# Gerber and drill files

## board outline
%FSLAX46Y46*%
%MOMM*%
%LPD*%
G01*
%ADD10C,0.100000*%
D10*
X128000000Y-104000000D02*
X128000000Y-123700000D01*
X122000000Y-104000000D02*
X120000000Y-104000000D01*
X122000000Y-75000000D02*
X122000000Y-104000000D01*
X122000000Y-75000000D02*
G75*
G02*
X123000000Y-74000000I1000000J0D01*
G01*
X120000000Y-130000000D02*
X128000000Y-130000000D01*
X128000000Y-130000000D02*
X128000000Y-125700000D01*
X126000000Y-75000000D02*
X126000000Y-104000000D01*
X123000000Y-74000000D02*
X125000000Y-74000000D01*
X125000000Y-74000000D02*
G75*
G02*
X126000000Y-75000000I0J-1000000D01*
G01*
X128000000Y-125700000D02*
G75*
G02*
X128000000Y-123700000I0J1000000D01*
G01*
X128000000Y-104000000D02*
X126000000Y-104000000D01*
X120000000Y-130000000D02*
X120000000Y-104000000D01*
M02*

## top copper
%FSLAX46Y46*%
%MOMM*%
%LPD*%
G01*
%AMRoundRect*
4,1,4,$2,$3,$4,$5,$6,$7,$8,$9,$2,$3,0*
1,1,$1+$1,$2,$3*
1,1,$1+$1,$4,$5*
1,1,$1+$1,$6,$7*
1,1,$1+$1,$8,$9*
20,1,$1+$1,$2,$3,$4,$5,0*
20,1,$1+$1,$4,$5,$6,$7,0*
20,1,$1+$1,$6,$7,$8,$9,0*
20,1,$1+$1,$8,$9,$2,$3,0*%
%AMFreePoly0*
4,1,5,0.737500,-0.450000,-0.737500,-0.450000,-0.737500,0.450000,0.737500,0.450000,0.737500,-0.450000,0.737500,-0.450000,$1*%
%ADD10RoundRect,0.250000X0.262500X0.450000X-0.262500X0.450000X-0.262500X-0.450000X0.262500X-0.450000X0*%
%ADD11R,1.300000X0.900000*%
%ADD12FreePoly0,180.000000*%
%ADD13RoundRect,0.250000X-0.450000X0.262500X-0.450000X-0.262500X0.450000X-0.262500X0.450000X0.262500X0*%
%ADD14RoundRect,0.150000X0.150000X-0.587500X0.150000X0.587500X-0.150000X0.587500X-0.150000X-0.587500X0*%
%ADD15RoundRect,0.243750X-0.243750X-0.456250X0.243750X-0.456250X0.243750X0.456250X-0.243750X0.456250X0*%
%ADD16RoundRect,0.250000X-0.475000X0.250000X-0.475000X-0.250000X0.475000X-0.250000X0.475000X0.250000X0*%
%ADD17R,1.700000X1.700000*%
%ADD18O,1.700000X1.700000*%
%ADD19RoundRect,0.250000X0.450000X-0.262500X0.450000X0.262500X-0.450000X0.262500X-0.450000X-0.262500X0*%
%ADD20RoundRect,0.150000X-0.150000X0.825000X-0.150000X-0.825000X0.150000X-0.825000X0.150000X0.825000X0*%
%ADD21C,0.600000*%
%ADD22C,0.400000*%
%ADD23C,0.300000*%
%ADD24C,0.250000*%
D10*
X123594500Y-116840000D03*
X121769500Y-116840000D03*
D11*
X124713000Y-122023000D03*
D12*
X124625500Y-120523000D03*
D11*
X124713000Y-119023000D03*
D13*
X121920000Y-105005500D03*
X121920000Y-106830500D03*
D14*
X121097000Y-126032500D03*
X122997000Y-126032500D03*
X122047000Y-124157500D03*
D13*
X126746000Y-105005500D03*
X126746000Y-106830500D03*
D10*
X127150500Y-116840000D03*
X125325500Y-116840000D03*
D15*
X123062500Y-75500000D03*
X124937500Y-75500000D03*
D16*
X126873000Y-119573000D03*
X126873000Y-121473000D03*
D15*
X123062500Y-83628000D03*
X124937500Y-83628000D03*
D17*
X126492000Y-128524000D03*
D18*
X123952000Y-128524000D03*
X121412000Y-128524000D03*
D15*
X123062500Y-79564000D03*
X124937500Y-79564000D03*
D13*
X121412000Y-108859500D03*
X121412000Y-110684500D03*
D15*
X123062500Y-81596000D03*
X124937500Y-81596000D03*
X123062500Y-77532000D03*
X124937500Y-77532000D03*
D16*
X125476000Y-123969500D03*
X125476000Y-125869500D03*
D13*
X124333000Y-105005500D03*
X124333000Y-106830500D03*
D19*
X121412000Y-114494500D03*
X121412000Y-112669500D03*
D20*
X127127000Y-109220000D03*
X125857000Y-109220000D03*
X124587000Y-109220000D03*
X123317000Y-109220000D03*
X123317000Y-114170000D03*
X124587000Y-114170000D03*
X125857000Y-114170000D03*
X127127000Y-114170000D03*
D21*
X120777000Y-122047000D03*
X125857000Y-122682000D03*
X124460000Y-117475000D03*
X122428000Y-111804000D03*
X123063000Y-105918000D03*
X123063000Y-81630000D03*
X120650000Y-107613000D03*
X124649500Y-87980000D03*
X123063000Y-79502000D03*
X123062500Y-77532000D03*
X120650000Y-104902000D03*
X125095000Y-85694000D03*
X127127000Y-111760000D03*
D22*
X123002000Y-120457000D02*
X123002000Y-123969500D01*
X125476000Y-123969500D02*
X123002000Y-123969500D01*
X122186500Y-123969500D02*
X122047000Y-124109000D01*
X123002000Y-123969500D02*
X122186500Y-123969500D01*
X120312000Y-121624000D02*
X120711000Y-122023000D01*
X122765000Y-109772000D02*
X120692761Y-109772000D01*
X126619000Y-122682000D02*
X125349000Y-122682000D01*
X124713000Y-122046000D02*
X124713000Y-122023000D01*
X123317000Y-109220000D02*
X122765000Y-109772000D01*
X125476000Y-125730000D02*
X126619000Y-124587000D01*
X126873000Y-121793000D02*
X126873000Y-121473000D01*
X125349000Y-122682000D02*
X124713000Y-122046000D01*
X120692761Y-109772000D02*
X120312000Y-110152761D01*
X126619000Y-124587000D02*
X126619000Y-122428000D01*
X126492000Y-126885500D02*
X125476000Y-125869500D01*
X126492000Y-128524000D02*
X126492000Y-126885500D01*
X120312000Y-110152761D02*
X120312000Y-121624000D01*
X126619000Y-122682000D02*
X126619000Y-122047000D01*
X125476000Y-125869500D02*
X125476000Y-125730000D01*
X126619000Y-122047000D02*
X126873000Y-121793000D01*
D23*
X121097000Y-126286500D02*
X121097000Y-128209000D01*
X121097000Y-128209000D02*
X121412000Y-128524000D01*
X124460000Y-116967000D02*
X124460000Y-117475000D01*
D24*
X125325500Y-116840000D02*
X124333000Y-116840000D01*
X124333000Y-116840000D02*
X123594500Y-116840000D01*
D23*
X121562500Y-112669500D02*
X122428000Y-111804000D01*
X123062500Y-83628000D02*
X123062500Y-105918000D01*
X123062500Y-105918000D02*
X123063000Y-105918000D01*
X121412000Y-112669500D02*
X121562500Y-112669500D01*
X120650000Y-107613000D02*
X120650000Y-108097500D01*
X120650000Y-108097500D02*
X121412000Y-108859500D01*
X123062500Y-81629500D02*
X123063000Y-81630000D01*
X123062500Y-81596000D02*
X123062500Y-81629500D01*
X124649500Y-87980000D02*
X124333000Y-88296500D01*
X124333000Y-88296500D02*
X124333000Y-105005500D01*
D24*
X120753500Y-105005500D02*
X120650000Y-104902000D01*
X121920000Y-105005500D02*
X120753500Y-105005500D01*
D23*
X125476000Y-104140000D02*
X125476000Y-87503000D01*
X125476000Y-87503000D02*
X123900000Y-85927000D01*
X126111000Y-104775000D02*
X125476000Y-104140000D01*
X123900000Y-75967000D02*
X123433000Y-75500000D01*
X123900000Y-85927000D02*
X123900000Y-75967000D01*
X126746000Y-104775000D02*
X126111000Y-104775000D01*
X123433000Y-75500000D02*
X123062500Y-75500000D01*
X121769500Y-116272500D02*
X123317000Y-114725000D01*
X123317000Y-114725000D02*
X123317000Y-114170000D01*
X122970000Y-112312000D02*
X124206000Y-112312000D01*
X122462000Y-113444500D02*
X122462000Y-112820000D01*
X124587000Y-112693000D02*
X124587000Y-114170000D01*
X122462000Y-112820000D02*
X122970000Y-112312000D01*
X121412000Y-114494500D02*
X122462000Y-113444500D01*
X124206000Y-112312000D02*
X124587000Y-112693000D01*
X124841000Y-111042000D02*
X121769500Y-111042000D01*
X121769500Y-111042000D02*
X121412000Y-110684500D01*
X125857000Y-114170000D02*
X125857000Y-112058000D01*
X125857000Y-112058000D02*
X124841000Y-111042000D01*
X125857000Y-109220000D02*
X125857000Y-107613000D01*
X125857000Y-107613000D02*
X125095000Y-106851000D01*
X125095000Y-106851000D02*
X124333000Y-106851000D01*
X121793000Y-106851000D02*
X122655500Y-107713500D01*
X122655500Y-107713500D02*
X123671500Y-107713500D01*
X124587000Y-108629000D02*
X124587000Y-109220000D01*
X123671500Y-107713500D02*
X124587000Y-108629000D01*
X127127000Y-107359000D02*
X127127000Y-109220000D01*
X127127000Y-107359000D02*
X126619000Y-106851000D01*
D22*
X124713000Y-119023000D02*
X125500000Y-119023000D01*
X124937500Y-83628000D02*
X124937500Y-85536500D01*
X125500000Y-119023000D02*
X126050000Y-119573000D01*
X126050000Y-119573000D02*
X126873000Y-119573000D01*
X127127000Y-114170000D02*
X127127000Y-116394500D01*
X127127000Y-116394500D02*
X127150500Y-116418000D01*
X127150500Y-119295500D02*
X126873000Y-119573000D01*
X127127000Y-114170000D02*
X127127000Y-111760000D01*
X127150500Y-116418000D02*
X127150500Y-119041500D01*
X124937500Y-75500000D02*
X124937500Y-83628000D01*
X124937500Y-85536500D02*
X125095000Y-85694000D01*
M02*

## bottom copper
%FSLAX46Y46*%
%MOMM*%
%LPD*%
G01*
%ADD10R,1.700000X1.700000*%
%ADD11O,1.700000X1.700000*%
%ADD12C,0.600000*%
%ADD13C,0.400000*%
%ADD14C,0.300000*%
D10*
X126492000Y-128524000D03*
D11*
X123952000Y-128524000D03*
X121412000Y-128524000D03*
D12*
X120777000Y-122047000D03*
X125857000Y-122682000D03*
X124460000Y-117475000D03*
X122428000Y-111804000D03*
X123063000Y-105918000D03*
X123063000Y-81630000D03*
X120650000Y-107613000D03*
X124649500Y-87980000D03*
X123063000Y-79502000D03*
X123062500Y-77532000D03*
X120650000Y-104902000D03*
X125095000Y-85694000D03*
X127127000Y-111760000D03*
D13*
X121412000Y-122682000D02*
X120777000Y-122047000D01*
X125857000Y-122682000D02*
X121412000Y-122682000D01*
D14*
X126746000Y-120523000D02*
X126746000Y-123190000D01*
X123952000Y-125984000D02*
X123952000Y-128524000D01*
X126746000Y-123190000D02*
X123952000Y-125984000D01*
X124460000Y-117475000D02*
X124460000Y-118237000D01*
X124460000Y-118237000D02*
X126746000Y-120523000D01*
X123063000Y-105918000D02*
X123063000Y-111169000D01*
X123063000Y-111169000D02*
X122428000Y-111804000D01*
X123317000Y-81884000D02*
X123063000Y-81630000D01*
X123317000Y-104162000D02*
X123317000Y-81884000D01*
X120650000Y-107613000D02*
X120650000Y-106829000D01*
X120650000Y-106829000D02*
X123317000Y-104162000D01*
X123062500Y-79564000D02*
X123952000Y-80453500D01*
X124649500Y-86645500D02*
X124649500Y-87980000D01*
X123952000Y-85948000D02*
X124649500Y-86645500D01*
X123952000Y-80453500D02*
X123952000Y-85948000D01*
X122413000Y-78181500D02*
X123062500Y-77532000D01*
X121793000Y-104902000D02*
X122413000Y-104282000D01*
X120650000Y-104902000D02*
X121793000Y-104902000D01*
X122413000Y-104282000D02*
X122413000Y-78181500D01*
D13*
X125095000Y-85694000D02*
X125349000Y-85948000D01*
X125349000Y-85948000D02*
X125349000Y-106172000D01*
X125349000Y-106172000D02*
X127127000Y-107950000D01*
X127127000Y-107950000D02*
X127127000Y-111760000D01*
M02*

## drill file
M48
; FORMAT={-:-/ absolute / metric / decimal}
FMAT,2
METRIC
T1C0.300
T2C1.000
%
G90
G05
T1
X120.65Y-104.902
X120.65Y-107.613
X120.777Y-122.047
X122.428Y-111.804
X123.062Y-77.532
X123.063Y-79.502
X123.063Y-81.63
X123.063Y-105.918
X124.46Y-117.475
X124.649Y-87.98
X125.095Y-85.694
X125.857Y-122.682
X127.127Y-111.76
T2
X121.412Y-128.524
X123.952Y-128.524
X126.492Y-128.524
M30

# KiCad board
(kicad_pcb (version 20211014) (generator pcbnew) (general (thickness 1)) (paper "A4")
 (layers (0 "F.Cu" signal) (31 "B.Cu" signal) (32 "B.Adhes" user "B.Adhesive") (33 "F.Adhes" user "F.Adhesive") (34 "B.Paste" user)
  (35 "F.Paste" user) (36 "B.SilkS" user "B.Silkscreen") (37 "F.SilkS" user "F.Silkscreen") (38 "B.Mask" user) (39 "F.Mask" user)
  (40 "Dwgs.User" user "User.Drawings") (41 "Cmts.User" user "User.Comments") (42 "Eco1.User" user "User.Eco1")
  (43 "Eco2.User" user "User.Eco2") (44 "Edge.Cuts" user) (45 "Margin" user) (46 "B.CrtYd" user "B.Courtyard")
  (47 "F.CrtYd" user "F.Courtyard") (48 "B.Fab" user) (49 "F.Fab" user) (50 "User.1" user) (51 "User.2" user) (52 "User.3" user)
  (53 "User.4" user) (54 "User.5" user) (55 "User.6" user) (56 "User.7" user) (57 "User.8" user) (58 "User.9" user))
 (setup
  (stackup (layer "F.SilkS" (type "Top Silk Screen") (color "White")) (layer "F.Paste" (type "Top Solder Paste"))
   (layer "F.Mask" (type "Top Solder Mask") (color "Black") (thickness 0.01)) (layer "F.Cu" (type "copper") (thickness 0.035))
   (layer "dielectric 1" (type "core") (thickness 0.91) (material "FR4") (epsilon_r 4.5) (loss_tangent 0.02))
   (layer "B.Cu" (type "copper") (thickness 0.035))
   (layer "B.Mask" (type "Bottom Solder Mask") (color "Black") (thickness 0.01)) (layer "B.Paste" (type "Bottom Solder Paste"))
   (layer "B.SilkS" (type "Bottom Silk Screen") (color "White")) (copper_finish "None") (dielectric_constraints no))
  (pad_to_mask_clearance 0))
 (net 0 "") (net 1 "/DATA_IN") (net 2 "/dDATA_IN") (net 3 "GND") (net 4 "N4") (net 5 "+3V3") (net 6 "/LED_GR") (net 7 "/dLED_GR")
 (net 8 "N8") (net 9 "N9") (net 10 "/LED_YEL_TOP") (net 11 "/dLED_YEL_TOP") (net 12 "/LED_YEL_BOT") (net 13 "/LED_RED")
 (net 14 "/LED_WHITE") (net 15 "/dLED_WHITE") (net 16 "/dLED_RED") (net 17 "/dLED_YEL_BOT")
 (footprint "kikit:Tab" (layer "F.Cu") (at 126.238 84.455 180)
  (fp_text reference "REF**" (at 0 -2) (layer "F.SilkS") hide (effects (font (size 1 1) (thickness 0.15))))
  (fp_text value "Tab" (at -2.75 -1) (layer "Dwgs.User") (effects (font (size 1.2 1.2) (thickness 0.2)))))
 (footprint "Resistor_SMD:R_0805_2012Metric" (layer "F.Cu") (at 122.682 116.84 180)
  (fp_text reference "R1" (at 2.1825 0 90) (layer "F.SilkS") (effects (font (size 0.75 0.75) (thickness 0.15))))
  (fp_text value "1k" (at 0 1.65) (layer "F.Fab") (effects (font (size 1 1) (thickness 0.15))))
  (pad "1" smd roundrect (at -0.9125 0 180) (size 1.025 1.4) (layers "F.Cu" "F.Paste" "F.Mask") (roundrect_rratio 0.243902)
   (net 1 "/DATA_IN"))
  (pad "2" smd roundrect (at 0.9125 0 180) (size 1.025 1.4) (layers "F.Cu" "F.Paste" "F.Mask") (roundrect_rratio 0.243902)
   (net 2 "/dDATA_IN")))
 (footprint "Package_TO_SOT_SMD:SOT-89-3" (layer "F.Cu") (at 123.063 120.523 180)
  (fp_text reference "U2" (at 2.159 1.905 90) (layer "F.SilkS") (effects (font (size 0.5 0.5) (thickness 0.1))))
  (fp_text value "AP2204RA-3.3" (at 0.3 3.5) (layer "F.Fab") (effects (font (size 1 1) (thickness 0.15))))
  (pad "1" smd rect (at -1.65 -1.5 180) (size 1.3 0.9) (layers "F.Cu" "F.Paste" "F.Mask") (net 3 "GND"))
  (pad "2" smd custom (at -1.5625 0 180) (size 1.475 0.9) (layers "F.Cu" "F.Paste" "F.Mask") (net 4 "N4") (zone_connect 2)
   (options (clearance outline) (anchor rect)) (primitives))
  (pad "3" smd rect (at -1.65 1.5 180) (size 1.3 0.9) (layers "F.Cu" "F.Paste" "F.Mask") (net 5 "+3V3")))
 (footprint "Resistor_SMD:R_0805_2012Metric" (layer "F.Cu") (at 121.92 105.918 -90)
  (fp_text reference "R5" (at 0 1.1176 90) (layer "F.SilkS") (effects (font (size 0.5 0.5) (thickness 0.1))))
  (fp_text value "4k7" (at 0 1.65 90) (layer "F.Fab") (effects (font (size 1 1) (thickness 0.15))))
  (pad "1" smd roundrect (at -0.9125 0 270) (size 1.025 1.4) (layers "F.Cu" "F.Paste" "F.Mask") (roundrect_rratio 0.243902)
   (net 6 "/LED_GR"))
  (pad "2" smd roundrect (at 0.9125 0 270) (size 1.025 1.4) (layers "F.Cu" "F.Paste" "F.Mask") (roundrect_rratio 0.243902)
   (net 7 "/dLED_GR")))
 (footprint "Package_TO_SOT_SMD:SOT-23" (layer "F.Cu") (at 122.047 125.095 90)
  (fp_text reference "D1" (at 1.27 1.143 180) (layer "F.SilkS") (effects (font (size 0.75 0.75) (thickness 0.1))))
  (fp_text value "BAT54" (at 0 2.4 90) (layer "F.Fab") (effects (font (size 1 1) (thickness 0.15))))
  (pad "1" smd roundrect (at -0.9375 -0.95 90) (size 1.475 0.6) (layers "F.Cu" "F.Paste" "F.Mask") (roundrect_rratio 0.25) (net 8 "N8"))
  (pad "2" smd roundrect (at -0.9375 0.95 90) (size 1.475 0.6) (layers "F.Cu" "F.Paste" "F.Mask") (roundrect_rratio 0.25) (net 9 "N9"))
  (pad "3" smd roundrect (at 0.9375 0 90) (size 1.475 0.6) (layers "F.Cu" "F.Paste" "F.Mask") (roundrect_rratio 0.25) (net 4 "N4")))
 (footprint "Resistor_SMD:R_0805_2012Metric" (layer "F.Cu") (at 126.746 105.918 -90)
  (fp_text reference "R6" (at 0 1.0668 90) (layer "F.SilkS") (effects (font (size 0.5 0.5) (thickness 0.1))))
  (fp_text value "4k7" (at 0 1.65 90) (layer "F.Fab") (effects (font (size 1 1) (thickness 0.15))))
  (pad "1" smd roundrect (at -0.9125 0 270) (size 1.025 1.4) (layers "F.Cu" "F.Paste" "F.Mask") (roundrect_rratio 0.243902)
   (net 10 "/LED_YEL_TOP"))
  (pad "2" smd roundrect (at 0.9125 0 270) (size 1.025 1.4) (layers "F.Cu" "F.Paste" "F.Mask") (roundrect_rratio 0.243902)
   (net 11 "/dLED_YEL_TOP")))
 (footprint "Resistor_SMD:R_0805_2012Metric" (layer "F.Cu") (at 126.238 116.84 180)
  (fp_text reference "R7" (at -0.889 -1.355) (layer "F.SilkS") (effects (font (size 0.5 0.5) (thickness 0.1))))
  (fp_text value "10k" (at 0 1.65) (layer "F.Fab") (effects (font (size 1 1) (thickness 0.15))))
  (pad "1" smd roundrect (at -0.9125 0 180) (size 1.025 1.4) (layers "F.Cu" "F.Paste" "F.Mask") (roundrect_rratio 0.243902) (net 5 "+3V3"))
  (pad "2" smd roundrect (at 0.9125 0 180) (size 1.025 1.4) (layers "F.Cu" "F.Paste" "F.Mask") (roundrect_rratio 0.243902)
   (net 1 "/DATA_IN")))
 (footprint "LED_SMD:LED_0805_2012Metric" (layer "F.Cu") (at 124 75.5)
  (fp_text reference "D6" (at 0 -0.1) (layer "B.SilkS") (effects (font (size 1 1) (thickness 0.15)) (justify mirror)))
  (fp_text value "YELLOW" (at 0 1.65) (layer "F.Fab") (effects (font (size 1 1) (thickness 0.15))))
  (pad "1" smd roundrect (at -0.9375 0) (size 0.975 1.4) (layers "F.Cu" "F.Paste" "F.Mask") (roundrect_rratio 0.25) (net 10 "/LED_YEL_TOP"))
  (pad "2" smd roundrect (at 0.9375 0) (size 0.975 1.4) (layers "F.Cu" "F.Paste" "F.Mask") (roundrect_rratio 0.25) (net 5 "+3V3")))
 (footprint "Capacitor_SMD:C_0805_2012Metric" (layer "F.Cu") (at 126.873 120.523 -90)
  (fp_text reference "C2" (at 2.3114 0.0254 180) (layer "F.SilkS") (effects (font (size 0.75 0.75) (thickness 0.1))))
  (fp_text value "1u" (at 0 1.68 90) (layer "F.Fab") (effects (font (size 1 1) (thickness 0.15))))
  (pad "1" smd roundrect (at -0.95 0 270) (size 1 1.45) (layers "F.Cu" "F.Paste" "F.Mask") (roundrect_rratio 0.25) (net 5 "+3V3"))
  (pad "2" smd roundrect (at 0.95 0 270) (size 1 1.45) (layers "F.Cu" "F.Paste" "F.Mask") (roundrect_rratio 0.25) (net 3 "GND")))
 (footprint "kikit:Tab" (layer "F.Cu") (at 128.27 115.697 180)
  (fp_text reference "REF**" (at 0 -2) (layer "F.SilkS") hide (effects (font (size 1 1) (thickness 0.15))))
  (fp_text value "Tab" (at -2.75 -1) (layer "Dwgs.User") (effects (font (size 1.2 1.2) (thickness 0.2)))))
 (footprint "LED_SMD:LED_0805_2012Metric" (layer "F.Cu") (at 124 83.628)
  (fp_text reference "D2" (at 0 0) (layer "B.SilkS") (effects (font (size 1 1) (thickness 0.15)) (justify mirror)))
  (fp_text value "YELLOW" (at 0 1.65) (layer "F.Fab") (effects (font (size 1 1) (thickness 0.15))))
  (pad "1" smd roundrect (at -0.9375 0) (size 0.975 1.4) (layers "F.Cu" "F.Paste" "F.Mask") (roundrect_rratio 0.25) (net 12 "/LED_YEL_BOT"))
  (pad "2" smd roundrect (at 0.9375 0) (size 0.975 1.4) (layers "F.Cu" "F.Paste" "F.Mask") (roundrect_rratio 0.25) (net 5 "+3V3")))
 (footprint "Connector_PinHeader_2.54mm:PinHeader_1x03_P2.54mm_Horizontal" (layer "F.Cu") (at 126.492 128.524 -90)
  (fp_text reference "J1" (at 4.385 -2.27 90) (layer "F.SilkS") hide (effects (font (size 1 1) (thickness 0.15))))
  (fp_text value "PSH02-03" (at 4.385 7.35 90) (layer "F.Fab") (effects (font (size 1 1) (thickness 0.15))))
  (pad "1" thru_hole rect (at 0 0 270) (size 1.7 1.7) (drill 1) (layers *.Cu *.Mask) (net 3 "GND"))
  (pad "2" thru_hole oval (at 0 2.54 270) (size 1.7 1.7) (drill 1) (layers *.Cu *.Mask) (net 1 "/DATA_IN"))
  (pad "3" thru_hole oval (at 0 5.08 270) (size 1.7 1.7) (drill 1) (layers *.Cu *.Mask) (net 8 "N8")))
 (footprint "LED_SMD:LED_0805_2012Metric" (layer "F.Cu") (at 124 79.564)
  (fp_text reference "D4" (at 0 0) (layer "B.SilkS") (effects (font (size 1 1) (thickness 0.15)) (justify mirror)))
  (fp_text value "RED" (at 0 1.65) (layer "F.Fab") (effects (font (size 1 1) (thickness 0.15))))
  (pad "1" smd roundrect (at -0.9375 0) (size 0.975 1.4) (layers "F.Cu" "F.Paste" "F.Mask") (roundrect_rratio 0.25) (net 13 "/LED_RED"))
  (pad "2" smd roundrect (at 0.9375 0) (size 0.975 1.4) (layers "F.Cu" "F.Paste" "F.Mask") (roundrect_rratio 0.25) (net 5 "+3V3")))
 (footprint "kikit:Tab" (layer "F.Cu") (at 121.793 84.455)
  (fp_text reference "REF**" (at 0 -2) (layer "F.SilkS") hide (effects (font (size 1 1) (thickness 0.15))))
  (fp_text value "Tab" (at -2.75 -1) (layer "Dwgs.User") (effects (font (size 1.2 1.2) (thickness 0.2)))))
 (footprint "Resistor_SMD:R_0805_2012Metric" (layer "F.Cu") (at 121.412 109.772 -90)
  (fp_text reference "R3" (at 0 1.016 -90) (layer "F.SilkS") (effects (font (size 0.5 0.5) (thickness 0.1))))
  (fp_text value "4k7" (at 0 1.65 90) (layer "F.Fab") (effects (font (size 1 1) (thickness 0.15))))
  (pad "1" smd roundrect (at -0.9125 0 270) (size 1.025 1.4) (layers "F.Cu" "F.Paste" "F.Mask") (roundrect_rratio 0.243902)
   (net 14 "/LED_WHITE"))
  (pad "2" smd roundrect (at 0.9125 0 270) (size 1.025 1.4) (layers "F.Cu" "F.Paste" "F.Mask") (roundrect_rratio 0.243902)
   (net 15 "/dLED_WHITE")))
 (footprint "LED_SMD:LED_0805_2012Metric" (layer "F.Cu") (at 124 81.596)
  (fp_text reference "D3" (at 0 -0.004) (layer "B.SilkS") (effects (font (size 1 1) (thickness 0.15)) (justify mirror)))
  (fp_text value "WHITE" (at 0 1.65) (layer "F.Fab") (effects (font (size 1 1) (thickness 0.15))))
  (pad "1" smd roundrect (at -0.9375 0) (size 0.975 1.4) (layers "F.Cu" "F.Paste" "F.Mask") (roundrect_rratio 0.25) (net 14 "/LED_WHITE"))
  (pad "2" smd roundrect (at 0.9375 0) (size 0.975 1.4) (layers "F.Cu" "F.Paste" "F.Mask") (roundrect_rratio 0.25) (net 5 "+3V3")))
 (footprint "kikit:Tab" (layer "F.Cu") (at 119.761 115.697)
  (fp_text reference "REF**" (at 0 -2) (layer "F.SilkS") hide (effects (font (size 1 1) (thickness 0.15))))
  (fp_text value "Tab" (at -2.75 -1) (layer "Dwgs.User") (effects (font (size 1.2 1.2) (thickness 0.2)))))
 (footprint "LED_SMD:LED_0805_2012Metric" (layer "F.Cu") (at 124 77.532)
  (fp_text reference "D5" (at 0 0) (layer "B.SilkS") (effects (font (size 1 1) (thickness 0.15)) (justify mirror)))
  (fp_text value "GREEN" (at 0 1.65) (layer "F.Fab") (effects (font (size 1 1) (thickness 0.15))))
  (pad "1" smd roundrect (at -0.9375 0) (size 0.975 1.4) (layers "F.Cu" "F.Paste" "F.Mask") (roundrect_rratio 0.25) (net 6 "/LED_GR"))
  (pad "2" smd roundrect (at 0.9375 0) (size 0.975 1.4) (layers "F.Cu" "F.Paste" "F.Mask") (roundrect_rratio 0.25) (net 5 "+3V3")))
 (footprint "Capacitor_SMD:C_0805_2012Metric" (layer "F.Cu") (at 125.476 124.9195 -90)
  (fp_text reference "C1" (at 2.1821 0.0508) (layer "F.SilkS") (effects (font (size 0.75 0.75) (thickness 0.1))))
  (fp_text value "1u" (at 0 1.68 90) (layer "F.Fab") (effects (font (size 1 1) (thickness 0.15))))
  (pad "1" smd roundrect (at -0.95 0 270) (size 1 1.45) (layers "F.Cu" "F.Paste" "F.Mask") (roundrect_rratio 0.25) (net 4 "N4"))
  (pad "2" smd roundrect (at 0.95 0 270) (size 1 1.45) (layers "F.Cu" "F.Paste" "F.Mask") (roundrect_rratio 0.25) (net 3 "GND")))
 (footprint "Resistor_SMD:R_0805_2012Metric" (layer "F.Cu") (at 124.333 105.918 -90)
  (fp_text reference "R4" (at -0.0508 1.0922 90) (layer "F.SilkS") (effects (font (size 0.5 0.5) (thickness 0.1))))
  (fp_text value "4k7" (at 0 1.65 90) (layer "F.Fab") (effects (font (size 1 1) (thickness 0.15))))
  (pad "1" smd roundrect (at -0.9125 0 270) (size 1.025 1.4) (layers "F.Cu" "F.Paste" "F.Mask") (roundrect_rratio 0.243902)
   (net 13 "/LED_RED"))
  (pad "2" smd roundrect (at 0.9125 0 270) (size 1.025 1.4) (layers "F.Cu" "F.Paste" "F.Mask") (roundrect_rratio 0.243902)
   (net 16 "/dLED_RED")))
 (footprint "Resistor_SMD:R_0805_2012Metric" (layer "F.Cu") (at 121.412 113.582 90)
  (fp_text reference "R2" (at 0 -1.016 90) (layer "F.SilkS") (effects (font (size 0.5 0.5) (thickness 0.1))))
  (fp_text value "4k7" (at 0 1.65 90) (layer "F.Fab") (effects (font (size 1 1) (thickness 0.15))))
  (pad "1" smd roundrect (at -0.9125 0 90) (size 1.025 1.4) (layers "F.Cu" "F.Paste" "F.Mask") (roundrect_rratio 0.243902)
   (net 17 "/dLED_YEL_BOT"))
  (pad "2" smd roundrect (at 0.9125 0 90) (size 1.025 1.4) (layers "F.Cu" "F.Paste" "F.Mask") (roundrect_rratio 0.243902)
   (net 12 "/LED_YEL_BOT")))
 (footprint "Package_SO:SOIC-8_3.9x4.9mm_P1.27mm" (layer "F.Cu") (at 125.222 111.695 -90)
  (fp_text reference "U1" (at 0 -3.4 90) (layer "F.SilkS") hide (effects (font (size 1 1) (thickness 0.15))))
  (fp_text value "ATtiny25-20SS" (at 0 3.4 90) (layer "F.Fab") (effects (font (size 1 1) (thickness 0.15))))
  (pad "1" smd roundrect (at -2.475 -1.905 270) (size 1.95 0.6) (layers "F.Cu" "F.Paste" "F.Mask") (roundrect_rratio 0.25)
   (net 11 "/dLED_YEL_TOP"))
  (pad "2" smd roundrect (at -2.475 -0.635 270) (size 1.95 0.6) (layers "F.Cu" "F.Paste" "F.Mask") (roundrect_rratio 0.25)
   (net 16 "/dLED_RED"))
  (pad "3" smd roundrect (at -2.475 0.635 270) (size 1.95 0.6) (layers "F.Cu" "F.Paste" "F.Mask") (roundrect_rratio 0.25) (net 7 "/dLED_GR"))
  (pad "4" smd roundrect (at -2.475 1.905 270) (size 1.95 0.6) (layers "F.Cu" "F.Paste" "F.Mask") (roundrect_rratio 0.25) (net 3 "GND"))
  (pad "5" smd roundrect (at 2.475 1.905 270) (size 1.95 0.6) (layers "F.Cu" "F.Paste" "F.Mask") (roundrect_rratio 0.25) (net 2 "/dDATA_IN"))
  (pad "6" smd roundrect (at 2.475 0.635 270) (size 1.95 0.6) (layers "F.Cu" "F.Paste" "F.Mask") (roundrect_rratio 0.25)
   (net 17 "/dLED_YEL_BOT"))
  (pad "7" smd roundrect (at 2.475 -0.635 270) (size 1.95 0.6) (layers "F.Cu" "F.Paste" "F.Mask") (roundrect_rratio 0.25)
   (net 15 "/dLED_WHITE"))
  (pad "8" smd roundrect (at 2.475 -1.905 270) (size 1.95 0.6) (layers "F.Cu" "F.Paste" "F.Mask") (roundrect_rratio 0.25) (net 5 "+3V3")))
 (gr_line (start 128 104) (end 128 123.7) (layer "Edge.Cuts") (width 0.1))
 (gr_line (start 122 104) (end 120 104) (layer "Edge.Cuts") (width 0.1))
 (gr_line (start 122 75) (end 122 104) (layer "Edge.Cuts") (width 0.1))
 (gr_arc (start 122 75) (mid 122.292893 74.292893) (end 123 74) (layer "Edge.Cuts") (width 0.1))
 (gr_line (start 120 130) (end 128 130) (layer "Edge.Cuts") (width 0.1))
 (gr_line (start 128 130) (end 128 125.7) (layer "Edge.Cuts") (width 0.1))
 (gr_line (start 126 75) (end 126 104) (layer "Edge.Cuts") (width 0.1))
 (gr_line (start 123 74) (end 125 74) (layer "Edge.Cuts") (width 0.1))
 (gr_arc (start 125 74) (mid 125.707107 74.292893) (end 126 75) (layer "Edge.Cuts") (width 0.1))
 (gr_arc (start 128 125.7) (mid 127 124.7) (end 128 123.7) (layer "Edge.Cuts") (width 0.1))
 (gr_line (start 128 104) (end 126 104) (layer "Edge.Cuts") (width 0.1))
 (gr_line (start 120 130) (end 120 104) (layer "Edge.Cuts") (width 0.1))
 (segment (start 123.002 120.457) (end 123.002 123.9695) (width 0.4) (layer "F.Cu") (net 4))
 (segment (start 125.476 123.9695) (end 123.002 123.9695) (width 0.4) (layer "F.Cu") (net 4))
 (segment (start 122.1865 123.9695) (end 122.047 124.109) (width 0.4) (layer "F.Cu") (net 4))
 (segment (start 123.002 123.9695) (end 122.1865 123.9695) (width 0.4) (layer "F.Cu") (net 4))
 (segment (start 120.312 121.624) (end 120.711 122.023) (width 0.4) (layer "F.Cu") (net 3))
 (segment (start 122.765 109.772) (end 120.692761 109.772) (width 0.4) (layer "F.Cu") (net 3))
 (segment (start 126.619 122.682) (end 125.349 122.682) (width 0.4) (layer "F.Cu") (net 3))
 (segment (start 124.713 122.046) (end 124.713 122.023) (width 0.4) (layer "F.Cu") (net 3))
 (segment (start 123.317 109.22) (end 122.765 109.772) (width 0.4) (layer "F.Cu") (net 3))
 (segment (start 125.476 125.73) (end 126.619 124.587) (width 0.4) (layer "F.Cu") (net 3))
 (segment (start 126.873 121.793) (end 126.873 121.473) (width 0.4) (layer "F.Cu") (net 3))
 (segment (start 125.349 122.682) (end 124.713 122.046) (width 0.4) (layer "F.Cu") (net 3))
 (segment (start 120.692761 109.772) (end 120.312 110.152761) (width 0.4) (layer "F.Cu") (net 3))
 (segment (start 126.619 124.587) (end 126.619 122.428) (width 0.4) (layer "F.Cu") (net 3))
 (segment (start 126.492 126.8855) (end 125.476 125.8695) (width 0.4) (layer "F.Cu") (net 3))
 (segment (start 126.492 128.524) (end 126.492 126.8855) (width 0.4) (layer "F.Cu") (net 3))
 (segment (start 120.312 110.152761) (end 120.312 121.624) (width 0.4) (layer "F.Cu") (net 3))
 (segment (start 126.619 122.682) (end 126.619 122.047) (width 0.4) (layer "F.Cu") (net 3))
 (segment (start 125.476 125.8695) (end 125.476 125.73) (width 0.4) (layer "F.Cu") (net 3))
 (segment (start 126.619 122.047) (end 126.873 121.793) (width 0.4) (layer "F.Cu") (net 3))
 (via (at 120.777 122.047) (size 0.6) (drill 0.3) (layers "F.Cu" "B.Cu") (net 3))
 (via (at 125.857 122.682) (size 0.6) (drill 0.3) (layers "F.Cu" "B.Cu") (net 3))
 (segment (start 121.412 122.682) (end 120.777 122.047) (width 0.4) (layer "B.Cu") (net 3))
 (segment (start 125.857 122.682) (end 121.412 122.682) (width 0.4) (layer "B.Cu") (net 3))
 (segment (start 121.097 126.2865) (end 121.097 128.209) (width 0.3) (layer "F.Cu") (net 8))
 (segment (start 121.097 128.209) (end 121.412 128.524) (width 0.3) (layer "F.Cu") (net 8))
 (segment (start 124.46 116.967) (end 124.46 117.475) (width 0.3) (layer "F.Cu") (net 1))
 (segment (start 125.3255 116.84) (end 124.333 116.84) (width 0.25) (layer "F.Cu") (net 1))
 (segment (start 124.333 116.84) (end 123.5945 116.84) (width 0.25) (layer "F.Cu") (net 1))
 (via (at 124.46 117.475) (size 0.6) (drill 0.3) (layers "F.Cu" "B.Cu") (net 1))
 (segment (start 126.746 120.523) (end 126.746 123.19) (width 0.3) (layer "B.Cu") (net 1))
 (segment (start 123.952 125.984) (end 123.952 128.524) (width 0.3) (layer "B.Cu") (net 1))
 (segment (start 126.746 123.19) (end 123.952 125.984) (width 0.3) (layer "B.Cu") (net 1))
 (segment (start 124.46 117.475) (end 124.46 118.237) (width 0.3) (layer "B.Cu") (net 1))
 (segment (start 124.46 118.237) (end 126.746 120.523) (width 0.3) (layer "B.Cu") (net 1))
 (segment (start 121.5625 112.6695) (end 122.428 111.804) (width 0.3) (layer "F.Cu") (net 12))
 (segment (start 123.0625 83.628) (end 123.0625 105.918) (width 0.3) (layer "F.Cu") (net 12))
 (segment (start 123.0625 105.918) (end 123.063 105.918) (width 0.3) (layer "F.Cu") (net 12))
 (segment (start 121.412 112.6695) (end 121.5625 112.6695) (width 0.3) (layer "F.Cu") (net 12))
 (via (at 122.428 111.804) (size 0.6) (drill 0.3) (layers "F.Cu" "B.Cu") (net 12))
 (via (at 123.063 105.918) (size 0.6) (drill 0.3) (layers "F.Cu" "B.Cu") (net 12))
 (segment (start 123.063 105.918) (end 123.063 111.169) (width 0.3) (layer "B.Cu") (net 12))
 (segment (start 123.063 111.169) (end 122.428 111.804) (width 0.3) (layer "B.Cu") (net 12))
 (segment (start 120.65 107.613) (end 120.65 108.0975) (width 0.3) (layer "F.Cu") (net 14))
 (segment (start 120.65 108.0975) (end 121.412 108.8595) (width 0.3) (layer "F.Cu") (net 14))
 (segment (start 123.0625 81.6295) (end 123.063 81.63) (width 0.3) (layer "F.Cu") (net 14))
 (segment (start 123.0625 81.596) (end 123.0625 81.6295) (width 0.3) (layer "F.Cu") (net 14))
 (via (at 123.063 81.63) (size 0.6) (drill 0.3) (layers "F.Cu" "B.Cu") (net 14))
 (via (at 120.65 107.613) (size 0.6) (drill 0.3) (layers "F.Cu" "B.Cu") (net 14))
 (segment (start 123.317 81.884) (end 123.063 81.63) (width 0.3) (layer "B.Cu") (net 14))
 (segment (start 123.317 104.162) (end 123.317 81.884) (width 0.3) (layer "B.Cu") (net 14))
 (segment (start 120.65 107.613) (end 120.65 106.829) (width 0.3) (layer "B.Cu") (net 14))
 (segment (start 120.65 106.829) (end 123.317 104.162) (width 0.3) (layer "B.Cu") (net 14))
 (segment (start 124.6495 87.98) (end 124.333 88.2965) (width 0.3) (layer "F.Cu") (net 13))
 (segment (start 124.333 88.2965) (end 124.333 105.0055) (width 0.3) (layer "F.Cu") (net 13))
 (via (at 124.6495 87.98) (size 0.6) (drill 0.3) (layers "F.Cu" "B.Cu") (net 13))
 (via (at 123.063 79.502) (size 0.6) (drill 0.3) (layers "F.Cu" "B.Cu") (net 13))
 (segment (start 123.0625 79.564) (end 123.952 80.4535) (width 0.3) (layer "B.Cu") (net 13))
 (segment (start 124.6495 86.6455) (end 124.6495 87.98) (width 0.3) (layer "B.Cu") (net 13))
 (segment (start 123.952 85.948) (end 124.6495 86.6455) (width 0.3) (layer "B.Cu") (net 13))
 (segment (start 123.952 80.4535) (end 123.952 85.948) (width 0.3) (layer "B.Cu") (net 13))
 (segment (start 120.7535 105.0055) (end 120.65 104.902) (width 0.25) (layer "F.Cu") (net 6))
 (segment (start 121.92 105.0055) (end 120.7535 105.0055) (width 0.25) (layer "F.Cu") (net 6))
 (via (at 123.0625 77.532) (size 0.6) (drill 0.3) (layers "F.Cu" "B.Cu") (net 6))
 (via (at 120.65 104.902) (size 0.6) (drill 0.3) (layers "F.Cu" "B.Cu") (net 6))
 (segment (start 122.413 78.1815) (end 123.0625 77.532) (width 0.3) (layer "B.Cu") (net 6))
 (segment (start 121.793 104.902) (end 122.413 104.282) (width 0.3) (layer "B.Cu") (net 6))
 (segment (start 120.65 104.902) (end 121.793 104.902) (width 0.3) (layer "B.Cu") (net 6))
 (segment (start 122.413 104.282) (end 122.413 78.1815) (width 0.3) (layer "B.Cu") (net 6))
 (segment (start 125.476 104.14) (end 125.476 87.503) (width 0.3) (layer "F.Cu") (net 10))
 (segment (start 125.476 87.503) (end 123.9 85.927) (width 0.3) (layer "F.Cu") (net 10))
 (segment (start 126.111 104.775) (end 125.476 104.14) (width 0.3) (layer "F.Cu") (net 10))
 (segment (start 123.9 75.967) (end 123.433 75.5) (width 0.3) (layer "F.Cu") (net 10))
 (segment (start 123.9 85.927) (end 123.9 75.967) (width 0.3) (layer "F.Cu") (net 10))
 (segment (start 126.746 104.775) (end 126.111 104.775) (width 0.3) (layer "F.Cu") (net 10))
 (segment (start 123.433 75.5) (end 123.0625 75.5) (width 0.3) (layer "F.Cu") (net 10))
 (segment (start 121.7695 116.2725) (end 123.317 114.725) (width 0.3) (layer "F.Cu") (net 2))
 (segment (start 123.317 114.725) (end 123.317 114.17) (width 0.3) (layer "F.Cu") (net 2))
 (segment (start 122.97 112.312) (end 124.206 112.312) (width 0.3) (layer "F.Cu") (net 17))
 (segment (start 122.462 113.4445) (end 122.462 112.82) (width 0.3) (layer "F.Cu") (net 17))
 (segment (start 124.587 112.693) (end 124.587 114.17) (width 0.3) (layer "F.Cu") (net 17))
 (segment (start 122.462 112.82) (end 122.97 112.312) (width 0.3) (layer "F.Cu") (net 17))
 (segment (start 121.412 114.4945) (end 122.462 113.4445) (width 0.3) (layer "F.Cu") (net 17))
 (segment (start 124.206 112.312) (end 124.587 112.693) (width 0.3) (layer "F.Cu") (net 17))
 (segment (start 124.841 111.042) (end 121.7695 111.042) (width 0.3) (layer "F.Cu") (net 15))
 (segment (start 121.7695 111.042) (end 121.412 110.6845) (width 0.3) (layer "F.Cu") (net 15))
 (segment (start 125.857 114.17) (end 125.857 112.058) (width 0.3) (layer "F.Cu") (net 15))
 (segment (start 125.857 112.058) (end 124.841 111.042) (width 0.3) (layer "F.Cu") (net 15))
 (segment (start 125.857 109.22) (end 125.857 107.613) (width 0.3) (layer "F.Cu") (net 16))
 (segment (start 125.857 107.613) (end 125.095 106.851) (width 0.3) (layer "F.Cu") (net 16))
 (segment (start 125.095 106.851) (end 124.333 106.851) (width 0.3) (layer "F.Cu") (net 16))
 (segment (start 121.793 106.851) (end 122.6555 107.7135) (width 0.3) (layer "F.Cu") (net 7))
 (segment (start 122.6555 107.7135) (end 123.6715 107.7135) (width 0.3) (layer "F.Cu") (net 7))
 (segment (start 124.587 108.629) (end 124.587 109.22) (width 0.3) (layer "F.Cu") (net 7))
 (segment (start 123.6715 107.7135) (end 124.587 108.629) (width 0.3) (layer "F.Cu") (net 7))
 (segment (start 127.127 107.359) (end 127.127 109.22) (width 0.3) (layer "F.Cu") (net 11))
 (segment (start 127.127 107.359) (end 126.619 106.851) (width 0.3) (layer "F.Cu") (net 11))
 (segment (start 124.713 119.023) (end 125.5 119.023) (width 0.4) (layer "F.Cu") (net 5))
 (segment (start 124.9375 83.628) (end 124.9375 85.5365) (width 0.4) (layer "F.Cu") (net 5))
 (segment (start 125.5 119.023) (end 126.05 119.573) (width 0.4) (layer "F.Cu") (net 5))
 (segment (start 126.05 119.573) (end 126.873 119.573) (width 0.4) (layer "F.Cu") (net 5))
 (segment (start 127.127 114.17) (end 127.127 116.3945) (width 0.4) (layer "F.Cu") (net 5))
 (segment (start 127.127 116.3945) (end 127.1505 116.418) (width 0.4) (layer "F.Cu") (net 5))
 (segment (start 127.1505 119.2955) (end 126.873 119.573) (width 0.4) (layer "F.Cu") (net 5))
 (segment (start 127.127 114.17) (end 127.127 111.76) (width 0.4) (layer "F.Cu") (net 5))
 (segment (start 127.1505 116.418) (end 127.1505 119.0415) (width 0.4) (layer "F.Cu") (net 5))
 (segment (start 124.9375 75.5) (end 124.9375 83.628) (width 0.4) (layer "F.Cu") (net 5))
 (segment (start 124.9375 85.5365) (end 125.095 85.694) (width 0.4) (layer "F.Cu") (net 5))
 (via (at 125.095 85.694) (size 0.6) (drill 0.3) (layers "F.Cu" "B.Cu") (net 5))
 (via (at 127.127 111.76) (size 0.6) (drill 0.3) (layers "F.Cu" "B.Cu") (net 5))
 (segment (start 125.095 85.694) (end 125.349 85.948) (width 0.4) (layer "B.Cu") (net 5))
 (segment (start 125.349 85.948) (end 125.349 106.172) (width 0.4) (layer "B.Cu") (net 5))
 (segment (start 125.349 106.172) (end 127.127 107.95) (width 0.4) (layer "B.Cu") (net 5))
 (segment (start 127.127 107.95) (end 127.127 111.76) (width 0.4) (layer "B.Cu") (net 5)))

